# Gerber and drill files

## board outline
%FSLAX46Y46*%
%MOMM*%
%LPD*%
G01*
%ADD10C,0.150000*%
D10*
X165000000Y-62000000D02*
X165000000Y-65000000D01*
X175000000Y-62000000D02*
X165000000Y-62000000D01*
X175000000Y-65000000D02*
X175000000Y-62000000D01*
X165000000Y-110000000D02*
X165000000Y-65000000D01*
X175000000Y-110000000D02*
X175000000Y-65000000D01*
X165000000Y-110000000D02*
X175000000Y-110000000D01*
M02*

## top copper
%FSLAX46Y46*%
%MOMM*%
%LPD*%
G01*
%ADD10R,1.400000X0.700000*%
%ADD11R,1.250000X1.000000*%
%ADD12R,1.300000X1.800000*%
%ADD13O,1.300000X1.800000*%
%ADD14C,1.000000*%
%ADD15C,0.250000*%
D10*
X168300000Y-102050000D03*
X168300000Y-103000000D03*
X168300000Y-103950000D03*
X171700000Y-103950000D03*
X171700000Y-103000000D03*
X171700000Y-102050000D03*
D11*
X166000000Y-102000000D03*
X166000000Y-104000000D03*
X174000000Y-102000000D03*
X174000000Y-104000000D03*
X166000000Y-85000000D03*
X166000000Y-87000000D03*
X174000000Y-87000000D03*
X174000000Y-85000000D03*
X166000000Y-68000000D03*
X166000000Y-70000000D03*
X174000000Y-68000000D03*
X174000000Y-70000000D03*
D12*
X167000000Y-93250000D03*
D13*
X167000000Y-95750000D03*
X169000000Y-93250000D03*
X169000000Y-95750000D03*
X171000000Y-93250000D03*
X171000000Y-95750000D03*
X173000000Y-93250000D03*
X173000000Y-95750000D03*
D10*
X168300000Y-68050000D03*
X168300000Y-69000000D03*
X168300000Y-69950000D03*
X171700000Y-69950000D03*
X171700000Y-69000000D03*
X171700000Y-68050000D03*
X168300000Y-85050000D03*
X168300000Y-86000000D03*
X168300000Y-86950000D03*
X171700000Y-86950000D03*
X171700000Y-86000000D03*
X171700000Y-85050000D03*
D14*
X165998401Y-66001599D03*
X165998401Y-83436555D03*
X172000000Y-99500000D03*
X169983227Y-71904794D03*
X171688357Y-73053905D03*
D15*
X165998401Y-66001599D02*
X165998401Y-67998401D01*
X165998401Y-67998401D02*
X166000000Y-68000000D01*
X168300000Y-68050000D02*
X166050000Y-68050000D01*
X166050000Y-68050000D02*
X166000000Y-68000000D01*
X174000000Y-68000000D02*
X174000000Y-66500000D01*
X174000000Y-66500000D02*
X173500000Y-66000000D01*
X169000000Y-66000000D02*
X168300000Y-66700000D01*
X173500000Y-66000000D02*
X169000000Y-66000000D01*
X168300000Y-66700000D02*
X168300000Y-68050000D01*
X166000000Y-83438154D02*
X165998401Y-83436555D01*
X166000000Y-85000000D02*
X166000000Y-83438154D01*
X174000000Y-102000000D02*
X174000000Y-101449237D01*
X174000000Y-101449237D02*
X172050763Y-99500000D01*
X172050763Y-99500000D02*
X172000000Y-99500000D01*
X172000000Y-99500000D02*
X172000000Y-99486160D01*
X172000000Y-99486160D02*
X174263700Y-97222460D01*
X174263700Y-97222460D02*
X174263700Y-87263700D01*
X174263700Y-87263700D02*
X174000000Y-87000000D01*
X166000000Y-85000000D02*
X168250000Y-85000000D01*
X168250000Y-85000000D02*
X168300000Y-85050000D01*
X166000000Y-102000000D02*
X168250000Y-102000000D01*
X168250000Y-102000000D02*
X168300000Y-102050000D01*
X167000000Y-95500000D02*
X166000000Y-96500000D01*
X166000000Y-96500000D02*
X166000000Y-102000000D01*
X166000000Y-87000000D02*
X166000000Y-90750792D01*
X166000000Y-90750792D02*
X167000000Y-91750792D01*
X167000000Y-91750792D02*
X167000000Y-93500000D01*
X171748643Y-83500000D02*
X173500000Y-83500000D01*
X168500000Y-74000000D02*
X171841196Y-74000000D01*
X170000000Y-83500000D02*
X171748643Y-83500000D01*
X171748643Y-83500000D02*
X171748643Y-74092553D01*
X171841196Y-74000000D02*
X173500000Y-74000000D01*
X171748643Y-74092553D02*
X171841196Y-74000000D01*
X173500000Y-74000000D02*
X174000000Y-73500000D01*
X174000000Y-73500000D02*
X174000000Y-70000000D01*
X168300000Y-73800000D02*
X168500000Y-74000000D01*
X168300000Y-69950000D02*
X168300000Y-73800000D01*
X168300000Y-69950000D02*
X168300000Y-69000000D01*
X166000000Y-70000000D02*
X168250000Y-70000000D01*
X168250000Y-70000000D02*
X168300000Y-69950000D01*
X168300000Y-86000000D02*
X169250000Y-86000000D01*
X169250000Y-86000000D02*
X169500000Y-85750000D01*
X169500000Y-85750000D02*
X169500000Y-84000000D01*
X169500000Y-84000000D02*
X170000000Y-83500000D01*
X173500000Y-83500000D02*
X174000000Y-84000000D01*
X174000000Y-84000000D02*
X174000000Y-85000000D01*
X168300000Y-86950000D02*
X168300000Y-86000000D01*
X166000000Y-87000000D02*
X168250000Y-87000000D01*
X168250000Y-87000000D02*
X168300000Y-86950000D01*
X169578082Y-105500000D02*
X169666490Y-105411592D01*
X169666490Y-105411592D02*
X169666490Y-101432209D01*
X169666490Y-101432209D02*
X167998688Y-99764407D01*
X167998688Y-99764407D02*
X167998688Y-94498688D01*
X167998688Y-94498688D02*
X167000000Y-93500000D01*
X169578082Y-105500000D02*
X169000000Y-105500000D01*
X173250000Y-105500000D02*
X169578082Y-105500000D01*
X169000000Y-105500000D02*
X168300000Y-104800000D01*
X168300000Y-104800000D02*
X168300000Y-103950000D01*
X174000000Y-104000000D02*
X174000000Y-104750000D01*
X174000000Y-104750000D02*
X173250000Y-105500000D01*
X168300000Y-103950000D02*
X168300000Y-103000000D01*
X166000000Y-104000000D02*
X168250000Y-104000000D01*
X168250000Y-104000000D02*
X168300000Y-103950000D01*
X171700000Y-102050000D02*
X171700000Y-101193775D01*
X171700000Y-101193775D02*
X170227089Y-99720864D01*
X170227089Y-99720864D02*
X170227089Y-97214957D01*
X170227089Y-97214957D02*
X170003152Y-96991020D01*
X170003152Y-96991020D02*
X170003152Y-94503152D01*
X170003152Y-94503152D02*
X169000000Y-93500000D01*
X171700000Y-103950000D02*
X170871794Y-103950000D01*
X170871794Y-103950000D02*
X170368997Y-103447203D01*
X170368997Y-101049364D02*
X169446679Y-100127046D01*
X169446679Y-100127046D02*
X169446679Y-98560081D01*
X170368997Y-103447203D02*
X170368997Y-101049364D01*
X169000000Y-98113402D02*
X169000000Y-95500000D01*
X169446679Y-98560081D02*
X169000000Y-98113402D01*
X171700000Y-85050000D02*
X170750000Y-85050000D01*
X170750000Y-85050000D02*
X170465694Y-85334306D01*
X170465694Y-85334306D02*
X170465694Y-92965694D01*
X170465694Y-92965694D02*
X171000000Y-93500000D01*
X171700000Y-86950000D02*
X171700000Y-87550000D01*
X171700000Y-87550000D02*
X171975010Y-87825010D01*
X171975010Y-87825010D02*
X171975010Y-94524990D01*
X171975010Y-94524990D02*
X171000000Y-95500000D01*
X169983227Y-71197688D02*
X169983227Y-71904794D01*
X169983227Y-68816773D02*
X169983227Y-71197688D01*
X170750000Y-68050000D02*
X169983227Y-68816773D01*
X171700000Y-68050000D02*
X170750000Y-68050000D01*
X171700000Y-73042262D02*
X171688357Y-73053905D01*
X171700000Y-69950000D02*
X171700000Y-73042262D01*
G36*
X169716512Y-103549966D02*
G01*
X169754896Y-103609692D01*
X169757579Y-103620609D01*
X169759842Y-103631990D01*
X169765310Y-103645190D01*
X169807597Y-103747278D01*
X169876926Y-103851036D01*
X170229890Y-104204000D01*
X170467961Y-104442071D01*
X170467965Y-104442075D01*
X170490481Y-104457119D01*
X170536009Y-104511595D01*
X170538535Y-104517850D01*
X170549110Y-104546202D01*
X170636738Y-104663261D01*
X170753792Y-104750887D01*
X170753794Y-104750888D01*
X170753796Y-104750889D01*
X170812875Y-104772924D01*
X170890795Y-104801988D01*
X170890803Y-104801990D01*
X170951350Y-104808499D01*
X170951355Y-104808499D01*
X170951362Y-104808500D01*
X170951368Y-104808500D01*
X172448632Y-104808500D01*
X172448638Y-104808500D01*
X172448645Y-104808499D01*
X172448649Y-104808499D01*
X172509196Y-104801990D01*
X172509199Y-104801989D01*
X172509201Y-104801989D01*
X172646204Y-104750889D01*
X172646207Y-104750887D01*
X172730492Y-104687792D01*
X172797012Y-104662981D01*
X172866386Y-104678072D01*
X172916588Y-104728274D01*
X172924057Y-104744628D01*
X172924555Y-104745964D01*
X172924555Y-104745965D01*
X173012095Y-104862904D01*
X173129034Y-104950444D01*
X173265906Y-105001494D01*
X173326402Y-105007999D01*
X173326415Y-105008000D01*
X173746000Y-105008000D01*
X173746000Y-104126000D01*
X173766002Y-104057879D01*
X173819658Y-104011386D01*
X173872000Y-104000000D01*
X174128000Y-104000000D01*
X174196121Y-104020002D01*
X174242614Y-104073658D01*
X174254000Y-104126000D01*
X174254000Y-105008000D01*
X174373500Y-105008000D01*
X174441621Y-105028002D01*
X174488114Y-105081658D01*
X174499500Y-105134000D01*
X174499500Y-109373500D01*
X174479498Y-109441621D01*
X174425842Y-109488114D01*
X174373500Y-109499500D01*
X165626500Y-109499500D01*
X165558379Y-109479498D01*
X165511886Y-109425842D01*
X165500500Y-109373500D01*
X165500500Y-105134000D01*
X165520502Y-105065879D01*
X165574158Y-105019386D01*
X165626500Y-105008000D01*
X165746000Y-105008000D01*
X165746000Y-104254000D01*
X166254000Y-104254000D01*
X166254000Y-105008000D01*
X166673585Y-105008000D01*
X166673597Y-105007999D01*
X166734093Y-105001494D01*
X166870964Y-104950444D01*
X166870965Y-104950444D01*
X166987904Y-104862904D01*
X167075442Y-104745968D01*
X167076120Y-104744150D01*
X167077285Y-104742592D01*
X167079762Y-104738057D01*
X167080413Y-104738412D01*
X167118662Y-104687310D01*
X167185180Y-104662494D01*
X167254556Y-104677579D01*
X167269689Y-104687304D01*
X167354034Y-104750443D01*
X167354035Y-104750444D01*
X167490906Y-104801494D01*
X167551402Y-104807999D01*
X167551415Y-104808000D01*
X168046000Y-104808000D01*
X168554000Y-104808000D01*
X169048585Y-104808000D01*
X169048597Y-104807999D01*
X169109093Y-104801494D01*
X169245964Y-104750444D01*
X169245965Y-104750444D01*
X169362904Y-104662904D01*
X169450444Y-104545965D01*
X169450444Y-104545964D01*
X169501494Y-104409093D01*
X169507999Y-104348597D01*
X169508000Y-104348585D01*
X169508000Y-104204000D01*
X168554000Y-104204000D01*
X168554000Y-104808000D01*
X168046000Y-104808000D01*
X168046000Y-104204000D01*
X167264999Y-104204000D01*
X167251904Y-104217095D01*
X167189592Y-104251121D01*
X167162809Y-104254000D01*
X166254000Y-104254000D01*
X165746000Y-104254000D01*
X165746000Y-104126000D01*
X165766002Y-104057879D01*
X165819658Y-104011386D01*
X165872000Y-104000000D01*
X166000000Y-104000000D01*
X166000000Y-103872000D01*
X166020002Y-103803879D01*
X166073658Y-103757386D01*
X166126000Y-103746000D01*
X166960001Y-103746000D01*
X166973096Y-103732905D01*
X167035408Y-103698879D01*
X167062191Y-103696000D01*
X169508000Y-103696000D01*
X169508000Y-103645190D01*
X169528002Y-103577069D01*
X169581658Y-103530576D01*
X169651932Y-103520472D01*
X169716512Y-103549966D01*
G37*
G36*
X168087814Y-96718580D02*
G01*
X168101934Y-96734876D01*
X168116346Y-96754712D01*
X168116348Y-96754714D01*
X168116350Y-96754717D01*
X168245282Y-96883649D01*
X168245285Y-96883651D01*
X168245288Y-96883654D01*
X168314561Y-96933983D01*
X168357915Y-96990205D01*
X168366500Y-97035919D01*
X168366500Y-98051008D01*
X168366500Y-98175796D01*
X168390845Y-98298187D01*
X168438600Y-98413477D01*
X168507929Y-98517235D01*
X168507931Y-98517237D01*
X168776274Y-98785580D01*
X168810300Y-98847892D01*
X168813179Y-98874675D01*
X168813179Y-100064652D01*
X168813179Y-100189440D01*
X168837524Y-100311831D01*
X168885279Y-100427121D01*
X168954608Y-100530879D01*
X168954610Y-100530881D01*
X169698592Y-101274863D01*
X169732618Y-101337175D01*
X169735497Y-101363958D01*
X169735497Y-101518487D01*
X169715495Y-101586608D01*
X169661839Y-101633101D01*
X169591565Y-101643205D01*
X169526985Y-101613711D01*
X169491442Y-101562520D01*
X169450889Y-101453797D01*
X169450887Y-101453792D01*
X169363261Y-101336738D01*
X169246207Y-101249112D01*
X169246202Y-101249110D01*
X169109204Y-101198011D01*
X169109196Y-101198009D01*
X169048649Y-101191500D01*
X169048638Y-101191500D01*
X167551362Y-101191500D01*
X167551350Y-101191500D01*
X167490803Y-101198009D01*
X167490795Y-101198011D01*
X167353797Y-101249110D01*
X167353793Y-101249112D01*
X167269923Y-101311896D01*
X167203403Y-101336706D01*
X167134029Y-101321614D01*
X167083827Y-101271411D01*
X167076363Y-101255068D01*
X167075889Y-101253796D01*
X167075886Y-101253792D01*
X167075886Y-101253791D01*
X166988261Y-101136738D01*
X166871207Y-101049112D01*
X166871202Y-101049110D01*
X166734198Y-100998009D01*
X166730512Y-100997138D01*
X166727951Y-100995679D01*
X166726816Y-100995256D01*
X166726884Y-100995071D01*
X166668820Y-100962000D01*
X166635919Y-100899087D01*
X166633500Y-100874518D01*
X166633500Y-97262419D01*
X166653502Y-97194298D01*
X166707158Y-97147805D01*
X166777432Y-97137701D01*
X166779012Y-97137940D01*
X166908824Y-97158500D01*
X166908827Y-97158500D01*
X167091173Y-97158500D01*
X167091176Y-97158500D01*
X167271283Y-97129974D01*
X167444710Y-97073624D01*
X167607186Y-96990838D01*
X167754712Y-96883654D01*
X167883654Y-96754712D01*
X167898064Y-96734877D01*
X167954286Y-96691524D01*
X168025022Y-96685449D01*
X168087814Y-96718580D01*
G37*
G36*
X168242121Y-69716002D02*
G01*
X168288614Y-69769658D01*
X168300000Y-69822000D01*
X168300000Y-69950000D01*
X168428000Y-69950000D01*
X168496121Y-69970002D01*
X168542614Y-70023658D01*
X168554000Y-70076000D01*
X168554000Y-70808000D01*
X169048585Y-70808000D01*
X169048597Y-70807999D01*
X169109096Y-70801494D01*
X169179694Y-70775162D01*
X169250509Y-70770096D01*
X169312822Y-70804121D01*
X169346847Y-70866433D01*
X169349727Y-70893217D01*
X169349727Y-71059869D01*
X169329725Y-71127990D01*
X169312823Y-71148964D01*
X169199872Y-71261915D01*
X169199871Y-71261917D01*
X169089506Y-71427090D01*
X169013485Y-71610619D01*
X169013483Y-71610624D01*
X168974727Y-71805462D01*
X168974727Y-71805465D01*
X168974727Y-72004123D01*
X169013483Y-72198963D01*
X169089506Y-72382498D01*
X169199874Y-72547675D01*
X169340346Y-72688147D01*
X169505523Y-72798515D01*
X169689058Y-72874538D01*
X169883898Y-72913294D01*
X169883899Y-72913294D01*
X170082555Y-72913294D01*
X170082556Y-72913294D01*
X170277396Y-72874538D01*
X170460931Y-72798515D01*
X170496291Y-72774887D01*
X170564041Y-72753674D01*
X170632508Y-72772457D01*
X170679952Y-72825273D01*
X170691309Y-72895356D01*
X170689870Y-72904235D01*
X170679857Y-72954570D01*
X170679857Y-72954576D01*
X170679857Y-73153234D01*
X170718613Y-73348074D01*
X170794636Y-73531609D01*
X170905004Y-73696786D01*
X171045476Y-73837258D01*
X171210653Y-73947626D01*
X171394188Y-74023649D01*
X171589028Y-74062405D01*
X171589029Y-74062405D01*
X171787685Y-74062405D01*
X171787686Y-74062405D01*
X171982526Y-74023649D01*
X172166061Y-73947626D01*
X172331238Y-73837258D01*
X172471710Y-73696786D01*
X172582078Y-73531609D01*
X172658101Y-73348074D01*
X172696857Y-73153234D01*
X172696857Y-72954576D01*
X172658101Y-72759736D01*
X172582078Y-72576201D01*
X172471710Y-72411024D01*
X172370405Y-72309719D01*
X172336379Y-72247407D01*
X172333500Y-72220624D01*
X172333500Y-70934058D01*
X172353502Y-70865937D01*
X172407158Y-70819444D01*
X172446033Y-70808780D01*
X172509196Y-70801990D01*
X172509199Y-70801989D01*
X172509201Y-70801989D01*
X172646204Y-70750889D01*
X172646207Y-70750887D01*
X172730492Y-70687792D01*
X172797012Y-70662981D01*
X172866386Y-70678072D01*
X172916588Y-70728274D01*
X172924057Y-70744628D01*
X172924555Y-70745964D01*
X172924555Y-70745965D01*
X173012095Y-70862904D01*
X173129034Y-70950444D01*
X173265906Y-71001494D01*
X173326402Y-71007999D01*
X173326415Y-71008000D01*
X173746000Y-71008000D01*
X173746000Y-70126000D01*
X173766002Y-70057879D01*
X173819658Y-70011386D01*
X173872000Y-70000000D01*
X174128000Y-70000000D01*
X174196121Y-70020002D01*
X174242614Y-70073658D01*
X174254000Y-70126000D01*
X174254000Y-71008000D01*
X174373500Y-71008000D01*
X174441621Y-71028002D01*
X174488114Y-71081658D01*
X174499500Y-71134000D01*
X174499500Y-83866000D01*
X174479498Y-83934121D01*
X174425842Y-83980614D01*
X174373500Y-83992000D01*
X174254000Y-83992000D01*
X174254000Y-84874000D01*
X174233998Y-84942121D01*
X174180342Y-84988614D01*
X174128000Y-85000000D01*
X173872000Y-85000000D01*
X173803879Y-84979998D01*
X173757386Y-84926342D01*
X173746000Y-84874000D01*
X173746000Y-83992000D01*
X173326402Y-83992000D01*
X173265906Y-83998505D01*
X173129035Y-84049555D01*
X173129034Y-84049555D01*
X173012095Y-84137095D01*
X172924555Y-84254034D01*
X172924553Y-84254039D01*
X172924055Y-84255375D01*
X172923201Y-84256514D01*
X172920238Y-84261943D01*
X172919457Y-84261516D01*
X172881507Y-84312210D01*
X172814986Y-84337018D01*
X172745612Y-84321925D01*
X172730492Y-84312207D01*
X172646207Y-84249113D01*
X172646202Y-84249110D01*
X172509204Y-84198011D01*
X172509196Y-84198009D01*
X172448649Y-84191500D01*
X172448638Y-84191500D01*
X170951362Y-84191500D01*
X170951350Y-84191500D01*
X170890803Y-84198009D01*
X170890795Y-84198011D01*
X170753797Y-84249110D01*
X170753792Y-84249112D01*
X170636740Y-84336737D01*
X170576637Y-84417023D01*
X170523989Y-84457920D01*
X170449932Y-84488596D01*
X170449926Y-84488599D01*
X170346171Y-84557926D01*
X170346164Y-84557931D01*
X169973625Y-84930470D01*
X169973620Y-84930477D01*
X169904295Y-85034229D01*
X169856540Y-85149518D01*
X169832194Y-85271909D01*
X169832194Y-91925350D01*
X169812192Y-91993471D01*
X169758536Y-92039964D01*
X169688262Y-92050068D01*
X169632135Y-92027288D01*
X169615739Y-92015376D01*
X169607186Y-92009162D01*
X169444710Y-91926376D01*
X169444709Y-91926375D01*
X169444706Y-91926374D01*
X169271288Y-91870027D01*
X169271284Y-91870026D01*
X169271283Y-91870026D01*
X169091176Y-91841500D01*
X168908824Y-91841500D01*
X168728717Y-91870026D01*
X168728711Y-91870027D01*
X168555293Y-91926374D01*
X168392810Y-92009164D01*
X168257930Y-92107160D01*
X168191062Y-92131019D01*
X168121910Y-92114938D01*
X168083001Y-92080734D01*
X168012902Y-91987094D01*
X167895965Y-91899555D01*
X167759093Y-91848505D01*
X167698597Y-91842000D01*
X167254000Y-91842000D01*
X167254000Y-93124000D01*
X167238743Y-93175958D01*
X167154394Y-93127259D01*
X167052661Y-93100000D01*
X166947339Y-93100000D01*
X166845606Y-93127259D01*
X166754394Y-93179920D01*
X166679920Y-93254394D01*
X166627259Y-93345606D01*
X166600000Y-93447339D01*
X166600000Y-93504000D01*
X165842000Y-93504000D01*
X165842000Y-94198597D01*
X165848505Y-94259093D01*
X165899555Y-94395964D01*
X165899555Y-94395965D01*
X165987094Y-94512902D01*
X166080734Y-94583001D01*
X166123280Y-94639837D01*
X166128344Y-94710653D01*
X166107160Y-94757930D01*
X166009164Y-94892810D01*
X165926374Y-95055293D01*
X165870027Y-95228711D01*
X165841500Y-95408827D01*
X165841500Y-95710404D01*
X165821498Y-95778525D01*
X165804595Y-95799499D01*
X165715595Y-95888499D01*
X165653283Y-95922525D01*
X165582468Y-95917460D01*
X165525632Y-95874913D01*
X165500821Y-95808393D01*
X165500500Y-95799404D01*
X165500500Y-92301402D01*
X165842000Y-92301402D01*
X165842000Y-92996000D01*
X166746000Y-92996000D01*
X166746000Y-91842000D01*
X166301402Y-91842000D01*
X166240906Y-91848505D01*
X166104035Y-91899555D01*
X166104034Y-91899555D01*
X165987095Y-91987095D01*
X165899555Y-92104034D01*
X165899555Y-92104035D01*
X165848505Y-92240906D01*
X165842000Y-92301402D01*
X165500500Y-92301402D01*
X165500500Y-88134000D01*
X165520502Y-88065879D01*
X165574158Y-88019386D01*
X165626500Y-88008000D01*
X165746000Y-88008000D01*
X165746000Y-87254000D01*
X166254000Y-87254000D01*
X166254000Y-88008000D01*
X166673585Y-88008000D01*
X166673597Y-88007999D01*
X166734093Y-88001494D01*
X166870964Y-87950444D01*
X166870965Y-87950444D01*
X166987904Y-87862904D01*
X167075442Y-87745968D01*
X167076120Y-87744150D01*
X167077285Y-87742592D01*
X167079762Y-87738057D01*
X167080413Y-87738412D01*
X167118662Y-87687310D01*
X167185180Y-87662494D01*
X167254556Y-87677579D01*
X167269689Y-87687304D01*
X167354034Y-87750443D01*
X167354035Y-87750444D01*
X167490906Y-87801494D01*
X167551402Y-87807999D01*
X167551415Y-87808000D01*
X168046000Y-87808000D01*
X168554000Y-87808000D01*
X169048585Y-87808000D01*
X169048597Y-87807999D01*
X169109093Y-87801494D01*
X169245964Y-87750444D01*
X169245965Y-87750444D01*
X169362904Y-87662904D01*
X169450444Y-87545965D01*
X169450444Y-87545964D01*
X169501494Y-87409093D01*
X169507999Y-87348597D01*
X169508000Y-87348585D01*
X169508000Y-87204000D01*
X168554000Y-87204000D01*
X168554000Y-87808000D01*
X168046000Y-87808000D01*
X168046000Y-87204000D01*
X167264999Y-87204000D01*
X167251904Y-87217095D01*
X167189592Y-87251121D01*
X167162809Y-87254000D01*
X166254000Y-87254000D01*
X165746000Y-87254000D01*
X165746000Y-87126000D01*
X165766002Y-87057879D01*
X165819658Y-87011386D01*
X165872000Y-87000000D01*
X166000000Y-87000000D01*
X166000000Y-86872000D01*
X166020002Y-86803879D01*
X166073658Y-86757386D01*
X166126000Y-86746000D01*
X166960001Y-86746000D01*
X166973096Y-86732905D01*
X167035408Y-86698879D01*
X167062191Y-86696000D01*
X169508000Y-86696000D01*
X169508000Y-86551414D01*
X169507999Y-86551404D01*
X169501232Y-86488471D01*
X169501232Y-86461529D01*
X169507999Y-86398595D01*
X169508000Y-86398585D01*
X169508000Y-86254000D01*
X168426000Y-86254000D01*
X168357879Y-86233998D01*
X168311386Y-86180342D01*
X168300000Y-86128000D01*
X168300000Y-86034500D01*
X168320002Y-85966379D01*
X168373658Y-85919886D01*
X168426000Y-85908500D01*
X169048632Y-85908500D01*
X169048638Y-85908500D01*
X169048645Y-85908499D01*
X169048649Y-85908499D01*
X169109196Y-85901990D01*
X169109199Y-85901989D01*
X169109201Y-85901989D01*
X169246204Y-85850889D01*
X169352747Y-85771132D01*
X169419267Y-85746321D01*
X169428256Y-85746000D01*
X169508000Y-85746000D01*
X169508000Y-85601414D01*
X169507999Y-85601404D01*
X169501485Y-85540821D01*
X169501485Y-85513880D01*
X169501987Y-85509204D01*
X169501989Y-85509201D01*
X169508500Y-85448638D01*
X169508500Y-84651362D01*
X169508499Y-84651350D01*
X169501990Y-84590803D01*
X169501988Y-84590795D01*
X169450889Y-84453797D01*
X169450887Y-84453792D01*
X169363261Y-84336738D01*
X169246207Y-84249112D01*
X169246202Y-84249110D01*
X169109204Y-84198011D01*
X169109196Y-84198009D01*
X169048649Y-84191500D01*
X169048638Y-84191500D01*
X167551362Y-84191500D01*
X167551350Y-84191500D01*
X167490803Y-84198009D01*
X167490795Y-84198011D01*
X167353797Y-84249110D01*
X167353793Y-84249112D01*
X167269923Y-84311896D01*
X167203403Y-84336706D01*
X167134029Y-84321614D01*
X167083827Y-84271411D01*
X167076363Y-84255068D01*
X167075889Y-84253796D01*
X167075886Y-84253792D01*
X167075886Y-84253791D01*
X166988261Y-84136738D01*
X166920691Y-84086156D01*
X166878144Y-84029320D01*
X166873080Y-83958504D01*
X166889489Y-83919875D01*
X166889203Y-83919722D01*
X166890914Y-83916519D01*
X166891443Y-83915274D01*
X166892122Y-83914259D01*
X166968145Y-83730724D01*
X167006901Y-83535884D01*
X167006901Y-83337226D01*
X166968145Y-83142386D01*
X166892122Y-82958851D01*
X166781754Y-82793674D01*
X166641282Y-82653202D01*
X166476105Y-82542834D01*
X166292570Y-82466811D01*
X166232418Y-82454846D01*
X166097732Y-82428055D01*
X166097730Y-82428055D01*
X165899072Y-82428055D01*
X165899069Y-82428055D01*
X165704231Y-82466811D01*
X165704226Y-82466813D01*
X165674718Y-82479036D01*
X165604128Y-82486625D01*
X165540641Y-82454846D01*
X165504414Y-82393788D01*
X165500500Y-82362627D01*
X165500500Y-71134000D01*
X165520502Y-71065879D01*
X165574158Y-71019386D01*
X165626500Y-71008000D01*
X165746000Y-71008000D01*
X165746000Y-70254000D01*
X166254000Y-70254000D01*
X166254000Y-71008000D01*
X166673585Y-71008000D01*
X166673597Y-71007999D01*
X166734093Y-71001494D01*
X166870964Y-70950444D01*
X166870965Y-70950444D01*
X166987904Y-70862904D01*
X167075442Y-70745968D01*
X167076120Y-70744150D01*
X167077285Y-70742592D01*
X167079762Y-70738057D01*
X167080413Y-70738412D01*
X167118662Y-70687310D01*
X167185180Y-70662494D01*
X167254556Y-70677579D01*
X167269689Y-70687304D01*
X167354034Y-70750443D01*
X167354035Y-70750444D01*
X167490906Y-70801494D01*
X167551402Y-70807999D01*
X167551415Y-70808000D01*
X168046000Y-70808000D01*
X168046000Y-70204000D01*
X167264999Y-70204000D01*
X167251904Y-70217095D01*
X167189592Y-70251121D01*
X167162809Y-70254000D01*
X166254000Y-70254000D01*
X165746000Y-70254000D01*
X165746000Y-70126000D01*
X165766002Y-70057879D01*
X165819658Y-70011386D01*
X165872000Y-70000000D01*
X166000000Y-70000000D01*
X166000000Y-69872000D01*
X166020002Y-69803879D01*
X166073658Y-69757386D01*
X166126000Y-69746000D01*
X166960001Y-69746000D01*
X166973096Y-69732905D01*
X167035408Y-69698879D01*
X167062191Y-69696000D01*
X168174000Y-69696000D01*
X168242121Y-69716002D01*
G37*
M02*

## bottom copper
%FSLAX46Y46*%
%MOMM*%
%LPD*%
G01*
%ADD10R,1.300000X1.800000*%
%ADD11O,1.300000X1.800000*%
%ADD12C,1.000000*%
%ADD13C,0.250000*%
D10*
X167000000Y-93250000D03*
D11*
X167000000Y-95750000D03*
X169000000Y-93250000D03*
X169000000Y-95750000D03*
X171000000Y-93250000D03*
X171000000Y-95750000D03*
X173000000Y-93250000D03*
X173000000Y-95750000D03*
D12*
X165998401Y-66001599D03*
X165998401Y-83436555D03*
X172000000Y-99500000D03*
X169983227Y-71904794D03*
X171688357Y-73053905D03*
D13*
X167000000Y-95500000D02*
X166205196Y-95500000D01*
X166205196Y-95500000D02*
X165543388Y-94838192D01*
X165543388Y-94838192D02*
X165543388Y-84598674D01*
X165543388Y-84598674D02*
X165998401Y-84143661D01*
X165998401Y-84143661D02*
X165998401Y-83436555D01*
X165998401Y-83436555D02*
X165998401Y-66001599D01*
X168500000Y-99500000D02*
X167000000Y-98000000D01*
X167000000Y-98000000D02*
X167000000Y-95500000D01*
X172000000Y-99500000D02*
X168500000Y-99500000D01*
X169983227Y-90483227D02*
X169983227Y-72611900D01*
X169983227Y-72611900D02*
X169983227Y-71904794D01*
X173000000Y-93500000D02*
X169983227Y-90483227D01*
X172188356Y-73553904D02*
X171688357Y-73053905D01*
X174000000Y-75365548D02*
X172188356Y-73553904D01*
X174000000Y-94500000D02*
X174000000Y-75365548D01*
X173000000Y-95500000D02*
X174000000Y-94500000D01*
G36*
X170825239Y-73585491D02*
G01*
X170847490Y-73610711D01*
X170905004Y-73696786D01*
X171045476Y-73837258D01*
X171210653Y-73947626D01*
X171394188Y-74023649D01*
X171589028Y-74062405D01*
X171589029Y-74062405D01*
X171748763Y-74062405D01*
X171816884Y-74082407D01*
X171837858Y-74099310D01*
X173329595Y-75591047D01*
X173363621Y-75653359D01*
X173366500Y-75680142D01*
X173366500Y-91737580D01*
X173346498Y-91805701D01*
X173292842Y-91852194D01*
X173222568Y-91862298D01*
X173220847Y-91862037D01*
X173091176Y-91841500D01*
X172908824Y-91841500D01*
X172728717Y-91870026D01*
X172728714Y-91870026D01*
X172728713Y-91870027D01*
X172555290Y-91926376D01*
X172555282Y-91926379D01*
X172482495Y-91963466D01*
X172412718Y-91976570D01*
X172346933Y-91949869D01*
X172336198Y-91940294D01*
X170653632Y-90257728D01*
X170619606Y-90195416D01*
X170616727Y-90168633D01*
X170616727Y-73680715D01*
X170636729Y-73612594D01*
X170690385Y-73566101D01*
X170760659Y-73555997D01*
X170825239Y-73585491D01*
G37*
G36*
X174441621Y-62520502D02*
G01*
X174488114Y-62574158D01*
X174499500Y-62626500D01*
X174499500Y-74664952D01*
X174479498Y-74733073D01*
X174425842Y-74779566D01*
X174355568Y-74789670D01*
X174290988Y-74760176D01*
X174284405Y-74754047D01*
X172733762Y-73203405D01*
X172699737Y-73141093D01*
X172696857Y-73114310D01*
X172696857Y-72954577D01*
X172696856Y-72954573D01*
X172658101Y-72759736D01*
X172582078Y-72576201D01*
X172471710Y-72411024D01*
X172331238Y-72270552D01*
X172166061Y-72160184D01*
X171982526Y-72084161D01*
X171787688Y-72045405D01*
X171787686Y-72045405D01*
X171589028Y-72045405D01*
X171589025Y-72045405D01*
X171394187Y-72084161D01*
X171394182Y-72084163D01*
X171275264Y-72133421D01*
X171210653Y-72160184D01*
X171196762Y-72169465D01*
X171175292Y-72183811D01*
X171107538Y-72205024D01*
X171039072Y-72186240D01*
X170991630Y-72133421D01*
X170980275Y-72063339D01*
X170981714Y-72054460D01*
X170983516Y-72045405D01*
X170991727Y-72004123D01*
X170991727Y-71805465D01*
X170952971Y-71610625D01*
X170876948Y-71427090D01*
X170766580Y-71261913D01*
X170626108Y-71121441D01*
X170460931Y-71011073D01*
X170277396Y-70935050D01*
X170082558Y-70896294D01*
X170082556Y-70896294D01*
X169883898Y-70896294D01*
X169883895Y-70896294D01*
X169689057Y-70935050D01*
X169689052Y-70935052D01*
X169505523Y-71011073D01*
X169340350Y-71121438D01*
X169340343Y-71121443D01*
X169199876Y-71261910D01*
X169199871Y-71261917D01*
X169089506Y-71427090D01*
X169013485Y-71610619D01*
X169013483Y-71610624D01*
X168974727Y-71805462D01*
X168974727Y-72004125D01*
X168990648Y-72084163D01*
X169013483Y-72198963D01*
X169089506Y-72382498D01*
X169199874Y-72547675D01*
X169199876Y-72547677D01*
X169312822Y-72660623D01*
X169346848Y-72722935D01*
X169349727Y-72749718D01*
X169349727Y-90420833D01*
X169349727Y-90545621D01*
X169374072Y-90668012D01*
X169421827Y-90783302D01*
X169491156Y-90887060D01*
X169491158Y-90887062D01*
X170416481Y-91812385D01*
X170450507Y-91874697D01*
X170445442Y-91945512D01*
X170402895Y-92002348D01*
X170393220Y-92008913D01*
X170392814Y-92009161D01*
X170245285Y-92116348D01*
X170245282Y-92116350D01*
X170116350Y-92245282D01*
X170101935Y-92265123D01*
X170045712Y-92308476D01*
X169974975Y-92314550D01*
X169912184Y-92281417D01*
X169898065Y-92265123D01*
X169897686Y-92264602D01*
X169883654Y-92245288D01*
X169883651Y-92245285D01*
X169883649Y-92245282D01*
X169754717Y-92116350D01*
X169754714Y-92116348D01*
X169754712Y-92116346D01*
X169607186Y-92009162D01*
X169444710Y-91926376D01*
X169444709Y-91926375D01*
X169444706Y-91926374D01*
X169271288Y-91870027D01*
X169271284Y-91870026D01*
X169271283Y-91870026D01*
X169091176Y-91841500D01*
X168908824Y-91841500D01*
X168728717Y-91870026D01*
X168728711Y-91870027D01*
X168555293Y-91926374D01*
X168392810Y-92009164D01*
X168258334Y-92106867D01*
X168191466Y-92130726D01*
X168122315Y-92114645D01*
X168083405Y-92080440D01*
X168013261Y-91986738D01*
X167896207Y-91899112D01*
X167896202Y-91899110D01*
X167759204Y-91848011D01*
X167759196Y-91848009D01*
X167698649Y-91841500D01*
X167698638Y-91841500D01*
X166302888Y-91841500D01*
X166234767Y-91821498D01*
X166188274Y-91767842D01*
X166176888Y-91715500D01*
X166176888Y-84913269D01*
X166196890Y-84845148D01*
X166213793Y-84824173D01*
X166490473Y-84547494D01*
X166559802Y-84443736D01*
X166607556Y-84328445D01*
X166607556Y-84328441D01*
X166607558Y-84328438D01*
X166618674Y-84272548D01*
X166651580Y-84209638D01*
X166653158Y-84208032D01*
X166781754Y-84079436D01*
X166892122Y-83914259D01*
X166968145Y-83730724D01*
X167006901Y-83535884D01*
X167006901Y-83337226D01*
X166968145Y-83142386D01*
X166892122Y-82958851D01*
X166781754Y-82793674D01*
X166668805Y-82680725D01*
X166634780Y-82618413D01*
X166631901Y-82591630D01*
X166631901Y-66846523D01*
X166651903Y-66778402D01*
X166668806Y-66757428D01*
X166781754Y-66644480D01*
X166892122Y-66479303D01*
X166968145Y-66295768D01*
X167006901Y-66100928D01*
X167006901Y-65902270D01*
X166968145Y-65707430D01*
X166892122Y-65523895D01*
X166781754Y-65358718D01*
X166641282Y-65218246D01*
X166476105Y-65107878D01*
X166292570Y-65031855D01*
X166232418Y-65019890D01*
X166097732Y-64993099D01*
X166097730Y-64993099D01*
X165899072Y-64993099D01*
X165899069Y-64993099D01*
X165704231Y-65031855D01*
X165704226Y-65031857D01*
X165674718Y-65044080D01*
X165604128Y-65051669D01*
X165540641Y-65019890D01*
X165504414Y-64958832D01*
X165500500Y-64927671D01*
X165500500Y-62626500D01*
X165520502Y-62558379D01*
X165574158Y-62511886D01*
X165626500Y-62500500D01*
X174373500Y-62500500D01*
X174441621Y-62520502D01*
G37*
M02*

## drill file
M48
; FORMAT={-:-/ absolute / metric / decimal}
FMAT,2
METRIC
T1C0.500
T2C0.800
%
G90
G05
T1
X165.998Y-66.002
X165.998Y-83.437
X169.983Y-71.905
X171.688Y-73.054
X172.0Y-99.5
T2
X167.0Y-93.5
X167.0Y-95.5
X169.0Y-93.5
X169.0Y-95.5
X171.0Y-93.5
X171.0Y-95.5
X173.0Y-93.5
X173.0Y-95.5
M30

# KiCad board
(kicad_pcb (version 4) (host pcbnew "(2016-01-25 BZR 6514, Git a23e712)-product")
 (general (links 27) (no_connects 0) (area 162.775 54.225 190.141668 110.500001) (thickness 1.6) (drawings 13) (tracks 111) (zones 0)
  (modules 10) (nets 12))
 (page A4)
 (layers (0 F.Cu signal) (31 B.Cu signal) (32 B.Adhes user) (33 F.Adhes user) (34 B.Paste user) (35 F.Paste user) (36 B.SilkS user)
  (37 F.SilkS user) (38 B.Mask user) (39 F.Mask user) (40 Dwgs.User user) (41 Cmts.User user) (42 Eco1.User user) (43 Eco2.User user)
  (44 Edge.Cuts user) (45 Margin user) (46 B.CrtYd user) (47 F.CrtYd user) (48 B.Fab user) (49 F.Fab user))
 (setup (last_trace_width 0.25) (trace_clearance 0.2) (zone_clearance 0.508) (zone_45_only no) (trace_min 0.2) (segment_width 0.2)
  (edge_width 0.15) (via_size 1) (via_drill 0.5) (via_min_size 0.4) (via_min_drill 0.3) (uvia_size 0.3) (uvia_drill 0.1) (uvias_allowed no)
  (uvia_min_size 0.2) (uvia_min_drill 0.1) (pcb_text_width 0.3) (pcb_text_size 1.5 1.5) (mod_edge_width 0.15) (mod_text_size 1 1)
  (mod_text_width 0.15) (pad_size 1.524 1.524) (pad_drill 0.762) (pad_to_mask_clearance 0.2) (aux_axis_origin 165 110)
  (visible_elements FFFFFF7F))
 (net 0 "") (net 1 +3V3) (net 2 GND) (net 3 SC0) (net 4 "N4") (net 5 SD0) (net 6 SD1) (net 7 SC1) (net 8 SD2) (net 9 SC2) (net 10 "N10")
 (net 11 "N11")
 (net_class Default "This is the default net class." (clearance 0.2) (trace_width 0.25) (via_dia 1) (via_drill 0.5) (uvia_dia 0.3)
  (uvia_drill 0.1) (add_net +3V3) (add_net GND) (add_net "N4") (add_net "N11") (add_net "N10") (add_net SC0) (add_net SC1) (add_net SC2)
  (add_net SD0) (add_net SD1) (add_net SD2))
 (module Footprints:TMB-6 (layer F.Cu) (at 170 103)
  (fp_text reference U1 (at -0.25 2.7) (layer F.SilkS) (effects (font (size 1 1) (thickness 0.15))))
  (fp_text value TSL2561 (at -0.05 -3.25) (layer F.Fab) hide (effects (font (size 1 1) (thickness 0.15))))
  (pad 1 smd rect (at -1.7 -0.95) (size 1.4 0.7) (layers F.Cu F.Paste F.Mask) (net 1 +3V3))
  (pad 2 smd rect (at -1.7 0) (size 1.4 0.7) (layers F.Cu F.Paste F.Mask) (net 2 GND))
  (pad 3 smd rect (at -1.7 0.95) (size 1.4 0.7) (layers F.Cu F.Paste F.Mask) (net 2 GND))
  (pad 4 smd rect (at 1.7 0.95) (size 1.4 0.7) (layers F.Cu F.Paste F.Mask) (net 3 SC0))
  (pad 5 smd rect (at 1.7 0) (size 1.4 0.7) (layers F.Cu F.Paste F.Mask) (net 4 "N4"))
  (pad 6 smd rect (at 1.7 -0.95) (size 1.4 0.7) (layers F.Cu F.Paste F.Mask) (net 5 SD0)))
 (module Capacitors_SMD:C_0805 (layer F.Cu) (at 166 103 270)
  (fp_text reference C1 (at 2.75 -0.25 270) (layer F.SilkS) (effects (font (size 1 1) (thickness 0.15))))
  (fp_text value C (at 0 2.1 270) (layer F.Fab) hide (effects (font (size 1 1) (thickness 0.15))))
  (pad 1 smd rect (at -1 0 270) (size 1 1.25) (layers F.Cu F.Paste F.Mask) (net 1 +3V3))
  (pad 2 smd rect (at 1 0 270) (size 1 1.25) (layers F.Cu F.Paste F.Mask) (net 2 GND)))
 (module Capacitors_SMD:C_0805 (layer F.Cu) (at 174 103 270)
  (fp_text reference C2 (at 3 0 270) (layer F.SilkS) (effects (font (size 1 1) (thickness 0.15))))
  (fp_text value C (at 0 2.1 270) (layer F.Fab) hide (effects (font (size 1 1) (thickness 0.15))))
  (pad 1 smd rect (at -1 0 270) (size 1 1.25) (layers F.Cu F.Paste F.Mask) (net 1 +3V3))
  (pad 2 smd rect (at 1 0 270) (size 1 1.25) (layers F.Cu F.Paste F.Mask) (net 2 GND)))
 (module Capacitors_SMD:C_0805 (layer F.Cu) (at 166 86 270)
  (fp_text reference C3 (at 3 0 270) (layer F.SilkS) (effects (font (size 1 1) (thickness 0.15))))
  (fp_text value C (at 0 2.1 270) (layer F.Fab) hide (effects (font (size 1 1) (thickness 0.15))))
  (pad 1 smd rect (at -1 0 270) (size 1 1.25) (layers F.Cu F.Paste F.Mask) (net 1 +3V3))
  (pad 2 smd rect (at 1 0 270) (size 1 1.25) (layers F.Cu F.Paste F.Mask) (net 2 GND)))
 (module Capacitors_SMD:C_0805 (layer F.Cu) (at 174 86 90)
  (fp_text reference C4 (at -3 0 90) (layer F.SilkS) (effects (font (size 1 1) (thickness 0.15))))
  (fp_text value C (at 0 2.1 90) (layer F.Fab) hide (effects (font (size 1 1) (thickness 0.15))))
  (pad 1 smd rect (at -1 0 90) (size 1 1.25) (layers F.Cu F.Paste F.Mask) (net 1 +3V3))
  (pad 2 smd rect (at 1 0 90) (size 1 1.25) (layers F.Cu F.Paste F.Mask) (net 2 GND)))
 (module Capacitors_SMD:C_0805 (layer F.Cu) (at 166 69 270)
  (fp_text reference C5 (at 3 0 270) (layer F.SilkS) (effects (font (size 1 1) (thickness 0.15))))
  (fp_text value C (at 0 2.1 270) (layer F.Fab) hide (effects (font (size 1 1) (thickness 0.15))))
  (pad 1 smd rect (at -1 0 270) (size 1 1.25) (layers F.Cu F.Paste F.Mask) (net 1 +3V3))
  (pad 2 smd rect (at 1 0 270) (size 1 1.25) (layers F.Cu F.Paste F.Mask) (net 2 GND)))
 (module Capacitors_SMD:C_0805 (layer F.Cu) (at 174 69 270)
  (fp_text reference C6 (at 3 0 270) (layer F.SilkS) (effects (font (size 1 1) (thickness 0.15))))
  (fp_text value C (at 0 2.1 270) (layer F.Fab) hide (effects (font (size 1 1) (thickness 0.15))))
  (pad 1 smd rect (at -1 0 270) (size 1 1.25) (layers F.Cu F.Paste F.Mask) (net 1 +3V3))
  (pad 2 smd rect (at 1 0 270) (size 1 1.25) (layers F.Cu F.Paste F.Mask) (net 2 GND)))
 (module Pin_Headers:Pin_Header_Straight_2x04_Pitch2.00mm (layer B.Cu) (at 170 94.5)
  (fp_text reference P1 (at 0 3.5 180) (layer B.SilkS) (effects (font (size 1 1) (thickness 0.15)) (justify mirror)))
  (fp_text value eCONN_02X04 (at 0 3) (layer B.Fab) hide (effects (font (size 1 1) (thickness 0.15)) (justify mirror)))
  (pad 1 thru_hole rect (at -3 -1) (size 1.3 1.8) (drill 0.8 (offset 0 -0.25)) (layers *.Cu *.Mask B.SilkS) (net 2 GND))
  (pad 2 thru_hole oval (at -3 1) (size 1.3 1.8) (drill 0.8 (offset 0 0.25)) (layers *.Cu *.Mask B.SilkS) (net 1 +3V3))
  (pad 3 thru_hole oval (at -1 -1) (size 1.3 1.8) (drill 0.8 (offset 0 -0.25)) (layers *.Cu *.Mask B.SilkS) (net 5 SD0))
  (pad 4 thru_hole oval (at -1 1) (size 1.3 1.8) (drill 0.8 (offset 0 0.25)) (layers *.Cu *.Mask B.SilkS) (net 3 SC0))
  (pad 5 thru_hole oval (at 1 -1) (size 1.3 1.8) (drill 0.8 (offset 0 -0.25)) (layers *.Cu *.Mask B.SilkS) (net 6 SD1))
  (pad 6 thru_hole oval (at 1 1) (size 1.3 1.8) (drill 0.8 (offset 0 0.25)) (layers *.Cu *.Mask B.SilkS) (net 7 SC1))
  (pad 7 thru_hole oval (at 3 -1) (size 1.3 1.8) (drill 0.8 (offset 0 -0.25)) (layers *.Cu *.Mask B.SilkS) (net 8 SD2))
  (pad 8 thru_hole oval (at 3 1) (size 1.3 1.8) (drill 0.8 (offset 0 0.25)) (layers *.Cu *.Mask B.SilkS) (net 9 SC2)))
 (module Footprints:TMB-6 (layer F.Cu) (at 170 69)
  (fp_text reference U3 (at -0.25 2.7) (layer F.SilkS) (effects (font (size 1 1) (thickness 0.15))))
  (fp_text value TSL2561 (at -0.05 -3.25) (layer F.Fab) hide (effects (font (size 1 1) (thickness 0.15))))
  (pad 1 smd rect (at -1.7 -0.95) (size 1.4 0.7) (layers F.Cu F.Paste F.Mask) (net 1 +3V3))
  (pad 2 smd rect (at -1.7 0) (size 1.4 0.7) (layers F.Cu F.Paste F.Mask) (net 2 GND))
  (pad 3 smd rect (at -1.7 0.95) (size 1.4 0.7) (layers F.Cu F.Paste F.Mask) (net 2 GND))
  (pad 4 smd rect (at 1.7 0.95) (size 1.4 0.7) (layers F.Cu F.Paste F.Mask) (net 9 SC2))
  (pad 5 smd rect (at 1.7 0) (size 1.4 0.7) (layers F.Cu F.Paste F.Mask) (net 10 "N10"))
  (pad 6 smd rect (at 1.7 -0.95) (size 1.4 0.7) (layers F.Cu F.Paste F.Mask) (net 8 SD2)))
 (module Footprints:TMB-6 (layer F.Cu) (at 170 86)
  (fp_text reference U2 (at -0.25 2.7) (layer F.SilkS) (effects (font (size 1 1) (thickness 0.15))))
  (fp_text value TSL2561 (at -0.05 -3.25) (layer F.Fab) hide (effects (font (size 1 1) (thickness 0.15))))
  (pad 1 smd rect (at -1.7 -0.95) (size 1.4 0.7) (layers F.Cu F.Paste F.Mask) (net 1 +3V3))
  (pad 2 smd rect (at -1.7 0) (size 1.4 0.7) (layers F.Cu F.Paste F.Mask) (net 2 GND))
  (pad 3 smd rect (at -1.7 0.95) (size 1.4 0.7) (layers F.Cu F.Paste F.Mask) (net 2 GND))
  (pad 4 smd rect (at 1.7 0.95) (size 1.4 0.7) (layers F.Cu F.Paste F.Mask) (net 7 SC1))
  (pad 5 smd rect (at 1.7 0) (size 1.4 0.7) (layers F.Cu F.Paste F.Mask) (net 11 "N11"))
  (pad 6 smd rect (at 1.7 -0.95) (size 1.4 0.7) (layers F.Cu F.Paste F.Mask) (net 6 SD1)))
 (gr_line (start 165 62) (end 165 65) (layer Edge.Cuts) (width 0.15))
 (gr_line (start 175 62) (end 165 62) (layer Edge.Cuts) (width 0.15))
 (gr_line (start 175 65) (end 175 62) (layer Edge.Cuts) (width 0.15))
 (gr_line (start 165 110) (end 165 65) (angle 90) (layer Edge.Cuts) (width 0.15))
 (gr_line (start 175 110) (end 175 65) (angle 90) (layer Edge.Cuts) (width 0.15))
 (gr_line (start 165 110) (end 175 110) (angle 90) (layer Edge.Cuts) (width 0.15))
 (segment (start 167 95.5) (end 166.205196 95.5) (width 0.25) (layer B.Cu) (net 1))
 (segment (start 166.205196 95.5) (end 165.543388 94.838192) (width 0.25) (layer B.Cu) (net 1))
 (segment (start 165.543388 94.838192) (end 165.543388 84.598674) (width 0.25) (layer B.Cu) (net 1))
 (segment (start 165.543388 84.598674) (end 165.998401 84.143661) (width 0.25) (layer B.Cu) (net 1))
 (segment (start 165.998401 84.143661) (end 165.998401 83.436555) (width 0.25) (layer B.Cu) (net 1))
 (segment (start 165.998401 66.001599) (end 165.998401 67.998401) (width 0.25) (layer F.Cu) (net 1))
 (segment (start 165.998401 67.998401) (end 166 68) (width 0.25) (layer F.Cu) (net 1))
 (via (at 165.998401 66.001599) (size 1) (drill 0.5) (layers F.Cu B.Cu) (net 1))
 (segment (start 165.998401 83.436555) (end 165.998401 66.001599) (width 0.25) (layer B.Cu) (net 1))
 (segment (start 168.3 68.05) (end 166.05 68.05) (width 0.25) (layer F.Cu) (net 1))
 (segment (start 166.05 68.05) (end 166 68) (width 0.25) (layer F.Cu) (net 1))
 (segment (start 174 68) (end 174 66.5) (width 0.25) (layer F.Cu) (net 1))
 (segment (start 174 66.5) (end 173.5 66) (width 0.25) (layer F.Cu) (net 1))
 (segment (start 169 66) (end 168.3 66.7) (width 0.25) (layer F.Cu) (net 1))
 (segment (start 173.5 66) (end 169 66) (width 0.25) (layer F.Cu) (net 1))
 (segment (start 168.3 66.7) (end 168.3 68.05) (width 0.25) (layer F.Cu) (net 1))
 (segment (start 166 83.438154) (end 165.998401 83.436555) (width 0.25) (layer F.Cu) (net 1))
 (segment (start 166 85) (end 166 83.438154) (width 0.25) (layer F.Cu) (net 1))
 (via (at 165.998401 83.436555) (size 1) (drill 0.5) (layers F.Cu B.Cu) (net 1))
 (segment (start 174 102) (end 174 101.449237) (width 0.25) (layer F.Cu) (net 1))
 (segment (start 174 101.449237) (end 172.050763 99.5) (width 0.25) (layer F.Cu) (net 1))
 (segment (start 172.050763 99.5) (end 172 99.5) (width 0.25) (layer F.Cu) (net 1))
 (segment (start 172 99.5) (end 172 99.48616) (width 0.25) (layer F.Cu) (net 1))
 (segment (start 172 99.48616) (end 174.2637 97.22246) (width 0.25) (layer F.Cu) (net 1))
 (segment (start 174.2637 97.22246) (end 174.2637 87.2637) (width 0.25) (layer F.Cu) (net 1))
 (segment (start 174.2637 87.2637) (end 174 87) (width 0.25) (layer F.Cu) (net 1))
 (segment (start 166 85) (end 168.25 85) (width 0.25) (layer F.Cu) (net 1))
 (segment (start 168.25 85) (end 168.3 85.05) (width 0.25) (layer F.Cu) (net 1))
 (segment (start 168.5 99.5) (end 167 98) (width 0.25) (layer B.Cu) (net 1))
 (segment (start 167 98) (end 167 95.5) (width 0.25) (layer B.Cu) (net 1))
 (segment (start 172 99.5) (end 168.5 99.5) (width 0.25) (layer B.Cu) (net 1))
 (via (at 172 99.5) (size 1) (drill 0.5) (layers F.Cu B.Cu) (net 1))
 (segment (start 166 102) (end 168.25 102) (width 0.25) (layer F.Cu) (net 1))
 (segment (start 168.25 102) (end 168.3 102.05) (width 0.25) (layer F.Cu) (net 1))
 (segment (start 167 95.5) (end 166 96.5) (width 0.25) (layer F.Cu) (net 1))
 (segment (start 166 96.5) (end 166 102) (width 0.25) (layer F.Cu) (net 1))
 (segment (start 166 87) (end 166 90.750792) (width 0.25) (layer F.Cu) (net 2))
 (segment (start 166 90.750792) (end 167 91.750792) (width 0.25) (layer F.Cu) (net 2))
 (segment (start 167 91.750792) (end 167 93.5) (width 0.25) (layer F.Cu) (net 2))
 (segment (start 171.748643 83.5) (end 173.5 83.5) (width 0.25) (layer F.Cu) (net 2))
 (segment (start 168.5 74) (end 171.841196 74) (width 0.25) (layer F.Cu) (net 2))
 (segment (start 170 83.5) (end 171.748643 83.5) (width 0.25) (layer F.Cu) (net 2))
 (segment (start 171.748643 83.5) (end 171.748643 74.092553) (width 0.25) (layer F.Cu) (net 2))
 (segment (start 171.841196 74) (end 173.5 74) (width 0.25) (layer F.Cu) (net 2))
 (segment (start 171.748643 74.092553) (end 171.841196 74) (width 0.25) (layer F.Cu) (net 2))
 (segment (start 173.5 74) (end 174 73.5) (width 0.25) (layer F.Cu) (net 2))
 (segment (start 174 73.5) (end 174 70) (width 0.25) (layer F.Cu) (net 2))
 (segment (start 168.3 73.8) (end 168.5 74) (width 0.25) (layer F.Cu) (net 2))
 (segment (start 168.3 69.95) (end 168.3 73.8) (width 0.25) (layer F.Cu) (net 2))
 (segment (start 168.3 69.95) (end 168.3 69) (width 0.25) (layer F.Cu) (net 2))
 (segment (start 166 70) (end 168.25 70) (width 0.25) (layer F.Cu) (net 2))
 (segment (start 168.25 70) (end 168.3 69.95) (width 0.25) (layer F.Cu) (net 2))
 (segment (start 168.3 86) (end 169.25 86) (width 0.25) (layer F.Cu) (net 2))
 (segment (start 169.25 86) (end 169.5 85.75) (width 0.25) (layer F.Cu) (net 2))
 (segment (start 169.5 85.75) (end 169.5 84) (width 0.25) (layer F.Cu) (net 2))
 (segment (start 169.5 84) (end 170 83.5) (width 0.25) (layer F.Cu) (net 2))
 (segment (start 173.5 83.5) (end 174 84) (width 0.25) (layer F.Cu) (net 2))
 (segment (start 174 84) (end 174 85) (width 0.25) (layer F.Cu) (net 2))
 (segment (start 168.3 86.95) (end 168.3 86) (width 0.25) (layer F.Cu) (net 2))
 (segment (start 166 87) (end 168.25 87) (width 0.25) (layer F.Cu) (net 2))
 (segment (start 168.25 87) (end 168.3 86.95) (width 0.25) (layer F.Cu) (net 2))
 (segment (start 169.578082 105.5) (end 169.66649 105.411592) (width 0.25) (layer F.Cu) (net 2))
 (segment (start 169.66649 105.411592) (end 169.66649 101.432209) (width 0.25) (layer F.Cu) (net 2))
 (segment (start 169.66649 101.432209) (end 167.998688 99.764407) (width 0.25) (layer F.Cu) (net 2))
 (segment (start 167.998688 99.764407) (end 167.998688 94.498688) (width 0.25) (layer F.Cu) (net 2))
 (segment (start 167.998688 94.498688) (end 167 93.5) (width 0.25) (layer F.Cu) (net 2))
 (segment (start 169.578082 105.5) (end 169 105.5) (width 0.25) (layer F.Cu) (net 2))
 (segment (start 173.25 105.5) (end 169.578082 105.5) (width 0.25) (layer F.Cu) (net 2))
 (segment (start 169 105.5) (end 168.3 104.8) (width 0.25) (layer F.Cu) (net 2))
 (segment (start 168.3 104.8) (end 168.3 103.95) (width 0.25) (layer F.Cu) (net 2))
 (segment (start 174 104) (end 174 104.75) (width 0.25) (layer F.Cu) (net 2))
 (segment (start 174 104.75) (end 173.25 105.5) (width 0.25) (layer F.Cu) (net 2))
 (segment (start 168.3 103.95) (end 168.3 103) (width 0.25) (layer F.Cu) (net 2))
 (segment (start 166 104) (end 168.25 104) (width 0.25) (layer F.Cu) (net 2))
 (segment (start 168.25 104) (end 168.3 103.95) (width 0.25) (layer F.Cu) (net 2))
 (segment (start 171.7 102.05) (end 171.7 101.193775) (width 0.25) (layer F.Cu) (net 5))
 (segment (start 171.7 101.193775) (end 170.227089 99.720864) (width 0.25) (layer F.Cu) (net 5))
 (segment (start 170.227089 99.720864) (end 170.227089 97.214957) (width 0.25) (layer F.Cu) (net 5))
 (segment (start 170.227089 97.214957) (end 170.003152 96.99102) (width 0.25) (layer F.Cu) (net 5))
 (segment (start 170.003152 96.99102) (end 170.003152 94.503152) (width 0.25) (layer F.Cu) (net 5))
 (segment (start 170.003152 94.503152) (end 169 93.5) (width 0.25) (layer F.Cu) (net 5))
 (segment (start 171.7 103.95) (end 170.871794 103.95) (width 0.25) (layer F.Cu) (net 3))
 (segment (start 170.871794 103.95) (end 170.368997 103.447203) (width 0.25) (layer F.Cu) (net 3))
 (segment (start 170.368997 101.049364) (end 169.446679 100.127046) (width 0.25) (layer F.Cu) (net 3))
 (segment (start 169.446679 100.127046) (end 169.446679 98.560081) (width 0.25) (layer F.Cu) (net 3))
 (segment (start 170.368997 103.447203) (end 170.368997 101.049364) (width 0.25) (layer F.Cu) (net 3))
 (segment (start 169 98.113402) (end 169 95.5) (width 0.25) (layer F.Cu) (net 3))
 (segment (start 169.446679 98.560081) (end 169 98.113402) (width 0.25) (layer F.Cu) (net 3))
 (segment (start 171.7 85.05) (end 170.75 85.05) (width 0.25) (layer F.Cu) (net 6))
 (segment (start 170.75 85.05) (end 170.465694 85.334306) (width 0.25) (layer F.Cu) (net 6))
 (segment (start 170.465694 85.334306) (end 170.465694 92.965694) (width 0.25) (layer F.Cu) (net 6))
 (segment (start 170.465694 92.965694) (end 171 93.5) (width 0.25) (layer F.Cu) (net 6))
 (segment (start 171.7 86.95) (end 171.7 87.55) (width 0.25) (layer F.Cu) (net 7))
 (segment (start 171.7 87.55) (end 171.97501 87.82501) (width 0.25) (layer F.Cu) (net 7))
 (segment (start 171.97501 87.82501) (end 171.97501 94.52499) (width 0.25) (layer F.Cu) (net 7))
 (segment (start 171.97501 94.52499) (end 171 95.5) (width 0.25) (layer F.Cu) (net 7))
 (segment (start 169.983227 71.197688) (end 169.983227 71.904794) (width 0.25) (layer F.Cu) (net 8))
 (segment (start 169.983227 68.816773) (end 169.983227 71.197688) (width 0.25) (layer F.Cu) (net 8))
 (segment (start 170.75 68.05) (end 169.983227 68.816773) (width 0.25) (layer F.Cu) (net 8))
 (segment (start 171.7 68.05) (end 170.75 68.05) (width 0.25) (layer F.Cu) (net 8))
 (segment (start 169.983227 90.483227) (end 169.983227 72.6119) (width 0.25) (layer B.Cu) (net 8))
 (segment (start 169.983227 72.6119) (end 169.983227 71.904794) (width 0.25) (layer B.Cu) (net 8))
 (segment (start 173 93.5) (end 169.983227 90.483227) (width 0.25) (layer B.Cu) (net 8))
 (via (at 169.983227 71.904794) (size 1) (drill 0.5) (layers F.Cu B.Cu) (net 8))
 (segment (start 172.188356 73.553904) (end 171.688357 73.053905) (width 0.25) (layer B.Cu) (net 9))
 (segment (start 174 75.365548) (end 172.188356 73.553904) (width 0.25) (layer B.Cu) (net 9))
 (segment (start 174 94.5) (end 174 75.365548) (width 0.25) (layer B.Cu) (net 9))
 (segment (start 173 95.5) (end 174 94.5) (width 0.25) (layer B.Cu) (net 9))
 (segment (start 171.7 73.042262) (end 171.688357 73.053905) (width 0.25) (layer F.Cu) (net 9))
 (segment (start 171.7 69.95) (end 171.7 73.042262) (width 0.25) (layer F.Cu) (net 9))
 (via (at 171.688357 73.053905) (size 1) (drill 0.5) (layers F.Cu B.Cu) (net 9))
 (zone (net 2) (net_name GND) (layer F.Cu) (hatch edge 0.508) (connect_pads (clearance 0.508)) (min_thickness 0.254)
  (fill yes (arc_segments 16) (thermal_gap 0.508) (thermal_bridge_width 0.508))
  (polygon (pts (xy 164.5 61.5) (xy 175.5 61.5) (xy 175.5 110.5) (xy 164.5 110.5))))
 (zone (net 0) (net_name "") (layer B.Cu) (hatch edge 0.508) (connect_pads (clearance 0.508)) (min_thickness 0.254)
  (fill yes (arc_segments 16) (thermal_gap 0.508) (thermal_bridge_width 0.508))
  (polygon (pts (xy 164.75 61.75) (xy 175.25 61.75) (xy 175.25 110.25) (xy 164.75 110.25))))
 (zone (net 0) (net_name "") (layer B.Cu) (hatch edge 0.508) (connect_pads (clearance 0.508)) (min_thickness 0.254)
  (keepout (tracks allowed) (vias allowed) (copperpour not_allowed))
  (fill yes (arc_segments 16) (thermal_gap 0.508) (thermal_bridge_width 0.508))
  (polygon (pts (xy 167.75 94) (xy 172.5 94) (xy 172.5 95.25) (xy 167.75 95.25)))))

